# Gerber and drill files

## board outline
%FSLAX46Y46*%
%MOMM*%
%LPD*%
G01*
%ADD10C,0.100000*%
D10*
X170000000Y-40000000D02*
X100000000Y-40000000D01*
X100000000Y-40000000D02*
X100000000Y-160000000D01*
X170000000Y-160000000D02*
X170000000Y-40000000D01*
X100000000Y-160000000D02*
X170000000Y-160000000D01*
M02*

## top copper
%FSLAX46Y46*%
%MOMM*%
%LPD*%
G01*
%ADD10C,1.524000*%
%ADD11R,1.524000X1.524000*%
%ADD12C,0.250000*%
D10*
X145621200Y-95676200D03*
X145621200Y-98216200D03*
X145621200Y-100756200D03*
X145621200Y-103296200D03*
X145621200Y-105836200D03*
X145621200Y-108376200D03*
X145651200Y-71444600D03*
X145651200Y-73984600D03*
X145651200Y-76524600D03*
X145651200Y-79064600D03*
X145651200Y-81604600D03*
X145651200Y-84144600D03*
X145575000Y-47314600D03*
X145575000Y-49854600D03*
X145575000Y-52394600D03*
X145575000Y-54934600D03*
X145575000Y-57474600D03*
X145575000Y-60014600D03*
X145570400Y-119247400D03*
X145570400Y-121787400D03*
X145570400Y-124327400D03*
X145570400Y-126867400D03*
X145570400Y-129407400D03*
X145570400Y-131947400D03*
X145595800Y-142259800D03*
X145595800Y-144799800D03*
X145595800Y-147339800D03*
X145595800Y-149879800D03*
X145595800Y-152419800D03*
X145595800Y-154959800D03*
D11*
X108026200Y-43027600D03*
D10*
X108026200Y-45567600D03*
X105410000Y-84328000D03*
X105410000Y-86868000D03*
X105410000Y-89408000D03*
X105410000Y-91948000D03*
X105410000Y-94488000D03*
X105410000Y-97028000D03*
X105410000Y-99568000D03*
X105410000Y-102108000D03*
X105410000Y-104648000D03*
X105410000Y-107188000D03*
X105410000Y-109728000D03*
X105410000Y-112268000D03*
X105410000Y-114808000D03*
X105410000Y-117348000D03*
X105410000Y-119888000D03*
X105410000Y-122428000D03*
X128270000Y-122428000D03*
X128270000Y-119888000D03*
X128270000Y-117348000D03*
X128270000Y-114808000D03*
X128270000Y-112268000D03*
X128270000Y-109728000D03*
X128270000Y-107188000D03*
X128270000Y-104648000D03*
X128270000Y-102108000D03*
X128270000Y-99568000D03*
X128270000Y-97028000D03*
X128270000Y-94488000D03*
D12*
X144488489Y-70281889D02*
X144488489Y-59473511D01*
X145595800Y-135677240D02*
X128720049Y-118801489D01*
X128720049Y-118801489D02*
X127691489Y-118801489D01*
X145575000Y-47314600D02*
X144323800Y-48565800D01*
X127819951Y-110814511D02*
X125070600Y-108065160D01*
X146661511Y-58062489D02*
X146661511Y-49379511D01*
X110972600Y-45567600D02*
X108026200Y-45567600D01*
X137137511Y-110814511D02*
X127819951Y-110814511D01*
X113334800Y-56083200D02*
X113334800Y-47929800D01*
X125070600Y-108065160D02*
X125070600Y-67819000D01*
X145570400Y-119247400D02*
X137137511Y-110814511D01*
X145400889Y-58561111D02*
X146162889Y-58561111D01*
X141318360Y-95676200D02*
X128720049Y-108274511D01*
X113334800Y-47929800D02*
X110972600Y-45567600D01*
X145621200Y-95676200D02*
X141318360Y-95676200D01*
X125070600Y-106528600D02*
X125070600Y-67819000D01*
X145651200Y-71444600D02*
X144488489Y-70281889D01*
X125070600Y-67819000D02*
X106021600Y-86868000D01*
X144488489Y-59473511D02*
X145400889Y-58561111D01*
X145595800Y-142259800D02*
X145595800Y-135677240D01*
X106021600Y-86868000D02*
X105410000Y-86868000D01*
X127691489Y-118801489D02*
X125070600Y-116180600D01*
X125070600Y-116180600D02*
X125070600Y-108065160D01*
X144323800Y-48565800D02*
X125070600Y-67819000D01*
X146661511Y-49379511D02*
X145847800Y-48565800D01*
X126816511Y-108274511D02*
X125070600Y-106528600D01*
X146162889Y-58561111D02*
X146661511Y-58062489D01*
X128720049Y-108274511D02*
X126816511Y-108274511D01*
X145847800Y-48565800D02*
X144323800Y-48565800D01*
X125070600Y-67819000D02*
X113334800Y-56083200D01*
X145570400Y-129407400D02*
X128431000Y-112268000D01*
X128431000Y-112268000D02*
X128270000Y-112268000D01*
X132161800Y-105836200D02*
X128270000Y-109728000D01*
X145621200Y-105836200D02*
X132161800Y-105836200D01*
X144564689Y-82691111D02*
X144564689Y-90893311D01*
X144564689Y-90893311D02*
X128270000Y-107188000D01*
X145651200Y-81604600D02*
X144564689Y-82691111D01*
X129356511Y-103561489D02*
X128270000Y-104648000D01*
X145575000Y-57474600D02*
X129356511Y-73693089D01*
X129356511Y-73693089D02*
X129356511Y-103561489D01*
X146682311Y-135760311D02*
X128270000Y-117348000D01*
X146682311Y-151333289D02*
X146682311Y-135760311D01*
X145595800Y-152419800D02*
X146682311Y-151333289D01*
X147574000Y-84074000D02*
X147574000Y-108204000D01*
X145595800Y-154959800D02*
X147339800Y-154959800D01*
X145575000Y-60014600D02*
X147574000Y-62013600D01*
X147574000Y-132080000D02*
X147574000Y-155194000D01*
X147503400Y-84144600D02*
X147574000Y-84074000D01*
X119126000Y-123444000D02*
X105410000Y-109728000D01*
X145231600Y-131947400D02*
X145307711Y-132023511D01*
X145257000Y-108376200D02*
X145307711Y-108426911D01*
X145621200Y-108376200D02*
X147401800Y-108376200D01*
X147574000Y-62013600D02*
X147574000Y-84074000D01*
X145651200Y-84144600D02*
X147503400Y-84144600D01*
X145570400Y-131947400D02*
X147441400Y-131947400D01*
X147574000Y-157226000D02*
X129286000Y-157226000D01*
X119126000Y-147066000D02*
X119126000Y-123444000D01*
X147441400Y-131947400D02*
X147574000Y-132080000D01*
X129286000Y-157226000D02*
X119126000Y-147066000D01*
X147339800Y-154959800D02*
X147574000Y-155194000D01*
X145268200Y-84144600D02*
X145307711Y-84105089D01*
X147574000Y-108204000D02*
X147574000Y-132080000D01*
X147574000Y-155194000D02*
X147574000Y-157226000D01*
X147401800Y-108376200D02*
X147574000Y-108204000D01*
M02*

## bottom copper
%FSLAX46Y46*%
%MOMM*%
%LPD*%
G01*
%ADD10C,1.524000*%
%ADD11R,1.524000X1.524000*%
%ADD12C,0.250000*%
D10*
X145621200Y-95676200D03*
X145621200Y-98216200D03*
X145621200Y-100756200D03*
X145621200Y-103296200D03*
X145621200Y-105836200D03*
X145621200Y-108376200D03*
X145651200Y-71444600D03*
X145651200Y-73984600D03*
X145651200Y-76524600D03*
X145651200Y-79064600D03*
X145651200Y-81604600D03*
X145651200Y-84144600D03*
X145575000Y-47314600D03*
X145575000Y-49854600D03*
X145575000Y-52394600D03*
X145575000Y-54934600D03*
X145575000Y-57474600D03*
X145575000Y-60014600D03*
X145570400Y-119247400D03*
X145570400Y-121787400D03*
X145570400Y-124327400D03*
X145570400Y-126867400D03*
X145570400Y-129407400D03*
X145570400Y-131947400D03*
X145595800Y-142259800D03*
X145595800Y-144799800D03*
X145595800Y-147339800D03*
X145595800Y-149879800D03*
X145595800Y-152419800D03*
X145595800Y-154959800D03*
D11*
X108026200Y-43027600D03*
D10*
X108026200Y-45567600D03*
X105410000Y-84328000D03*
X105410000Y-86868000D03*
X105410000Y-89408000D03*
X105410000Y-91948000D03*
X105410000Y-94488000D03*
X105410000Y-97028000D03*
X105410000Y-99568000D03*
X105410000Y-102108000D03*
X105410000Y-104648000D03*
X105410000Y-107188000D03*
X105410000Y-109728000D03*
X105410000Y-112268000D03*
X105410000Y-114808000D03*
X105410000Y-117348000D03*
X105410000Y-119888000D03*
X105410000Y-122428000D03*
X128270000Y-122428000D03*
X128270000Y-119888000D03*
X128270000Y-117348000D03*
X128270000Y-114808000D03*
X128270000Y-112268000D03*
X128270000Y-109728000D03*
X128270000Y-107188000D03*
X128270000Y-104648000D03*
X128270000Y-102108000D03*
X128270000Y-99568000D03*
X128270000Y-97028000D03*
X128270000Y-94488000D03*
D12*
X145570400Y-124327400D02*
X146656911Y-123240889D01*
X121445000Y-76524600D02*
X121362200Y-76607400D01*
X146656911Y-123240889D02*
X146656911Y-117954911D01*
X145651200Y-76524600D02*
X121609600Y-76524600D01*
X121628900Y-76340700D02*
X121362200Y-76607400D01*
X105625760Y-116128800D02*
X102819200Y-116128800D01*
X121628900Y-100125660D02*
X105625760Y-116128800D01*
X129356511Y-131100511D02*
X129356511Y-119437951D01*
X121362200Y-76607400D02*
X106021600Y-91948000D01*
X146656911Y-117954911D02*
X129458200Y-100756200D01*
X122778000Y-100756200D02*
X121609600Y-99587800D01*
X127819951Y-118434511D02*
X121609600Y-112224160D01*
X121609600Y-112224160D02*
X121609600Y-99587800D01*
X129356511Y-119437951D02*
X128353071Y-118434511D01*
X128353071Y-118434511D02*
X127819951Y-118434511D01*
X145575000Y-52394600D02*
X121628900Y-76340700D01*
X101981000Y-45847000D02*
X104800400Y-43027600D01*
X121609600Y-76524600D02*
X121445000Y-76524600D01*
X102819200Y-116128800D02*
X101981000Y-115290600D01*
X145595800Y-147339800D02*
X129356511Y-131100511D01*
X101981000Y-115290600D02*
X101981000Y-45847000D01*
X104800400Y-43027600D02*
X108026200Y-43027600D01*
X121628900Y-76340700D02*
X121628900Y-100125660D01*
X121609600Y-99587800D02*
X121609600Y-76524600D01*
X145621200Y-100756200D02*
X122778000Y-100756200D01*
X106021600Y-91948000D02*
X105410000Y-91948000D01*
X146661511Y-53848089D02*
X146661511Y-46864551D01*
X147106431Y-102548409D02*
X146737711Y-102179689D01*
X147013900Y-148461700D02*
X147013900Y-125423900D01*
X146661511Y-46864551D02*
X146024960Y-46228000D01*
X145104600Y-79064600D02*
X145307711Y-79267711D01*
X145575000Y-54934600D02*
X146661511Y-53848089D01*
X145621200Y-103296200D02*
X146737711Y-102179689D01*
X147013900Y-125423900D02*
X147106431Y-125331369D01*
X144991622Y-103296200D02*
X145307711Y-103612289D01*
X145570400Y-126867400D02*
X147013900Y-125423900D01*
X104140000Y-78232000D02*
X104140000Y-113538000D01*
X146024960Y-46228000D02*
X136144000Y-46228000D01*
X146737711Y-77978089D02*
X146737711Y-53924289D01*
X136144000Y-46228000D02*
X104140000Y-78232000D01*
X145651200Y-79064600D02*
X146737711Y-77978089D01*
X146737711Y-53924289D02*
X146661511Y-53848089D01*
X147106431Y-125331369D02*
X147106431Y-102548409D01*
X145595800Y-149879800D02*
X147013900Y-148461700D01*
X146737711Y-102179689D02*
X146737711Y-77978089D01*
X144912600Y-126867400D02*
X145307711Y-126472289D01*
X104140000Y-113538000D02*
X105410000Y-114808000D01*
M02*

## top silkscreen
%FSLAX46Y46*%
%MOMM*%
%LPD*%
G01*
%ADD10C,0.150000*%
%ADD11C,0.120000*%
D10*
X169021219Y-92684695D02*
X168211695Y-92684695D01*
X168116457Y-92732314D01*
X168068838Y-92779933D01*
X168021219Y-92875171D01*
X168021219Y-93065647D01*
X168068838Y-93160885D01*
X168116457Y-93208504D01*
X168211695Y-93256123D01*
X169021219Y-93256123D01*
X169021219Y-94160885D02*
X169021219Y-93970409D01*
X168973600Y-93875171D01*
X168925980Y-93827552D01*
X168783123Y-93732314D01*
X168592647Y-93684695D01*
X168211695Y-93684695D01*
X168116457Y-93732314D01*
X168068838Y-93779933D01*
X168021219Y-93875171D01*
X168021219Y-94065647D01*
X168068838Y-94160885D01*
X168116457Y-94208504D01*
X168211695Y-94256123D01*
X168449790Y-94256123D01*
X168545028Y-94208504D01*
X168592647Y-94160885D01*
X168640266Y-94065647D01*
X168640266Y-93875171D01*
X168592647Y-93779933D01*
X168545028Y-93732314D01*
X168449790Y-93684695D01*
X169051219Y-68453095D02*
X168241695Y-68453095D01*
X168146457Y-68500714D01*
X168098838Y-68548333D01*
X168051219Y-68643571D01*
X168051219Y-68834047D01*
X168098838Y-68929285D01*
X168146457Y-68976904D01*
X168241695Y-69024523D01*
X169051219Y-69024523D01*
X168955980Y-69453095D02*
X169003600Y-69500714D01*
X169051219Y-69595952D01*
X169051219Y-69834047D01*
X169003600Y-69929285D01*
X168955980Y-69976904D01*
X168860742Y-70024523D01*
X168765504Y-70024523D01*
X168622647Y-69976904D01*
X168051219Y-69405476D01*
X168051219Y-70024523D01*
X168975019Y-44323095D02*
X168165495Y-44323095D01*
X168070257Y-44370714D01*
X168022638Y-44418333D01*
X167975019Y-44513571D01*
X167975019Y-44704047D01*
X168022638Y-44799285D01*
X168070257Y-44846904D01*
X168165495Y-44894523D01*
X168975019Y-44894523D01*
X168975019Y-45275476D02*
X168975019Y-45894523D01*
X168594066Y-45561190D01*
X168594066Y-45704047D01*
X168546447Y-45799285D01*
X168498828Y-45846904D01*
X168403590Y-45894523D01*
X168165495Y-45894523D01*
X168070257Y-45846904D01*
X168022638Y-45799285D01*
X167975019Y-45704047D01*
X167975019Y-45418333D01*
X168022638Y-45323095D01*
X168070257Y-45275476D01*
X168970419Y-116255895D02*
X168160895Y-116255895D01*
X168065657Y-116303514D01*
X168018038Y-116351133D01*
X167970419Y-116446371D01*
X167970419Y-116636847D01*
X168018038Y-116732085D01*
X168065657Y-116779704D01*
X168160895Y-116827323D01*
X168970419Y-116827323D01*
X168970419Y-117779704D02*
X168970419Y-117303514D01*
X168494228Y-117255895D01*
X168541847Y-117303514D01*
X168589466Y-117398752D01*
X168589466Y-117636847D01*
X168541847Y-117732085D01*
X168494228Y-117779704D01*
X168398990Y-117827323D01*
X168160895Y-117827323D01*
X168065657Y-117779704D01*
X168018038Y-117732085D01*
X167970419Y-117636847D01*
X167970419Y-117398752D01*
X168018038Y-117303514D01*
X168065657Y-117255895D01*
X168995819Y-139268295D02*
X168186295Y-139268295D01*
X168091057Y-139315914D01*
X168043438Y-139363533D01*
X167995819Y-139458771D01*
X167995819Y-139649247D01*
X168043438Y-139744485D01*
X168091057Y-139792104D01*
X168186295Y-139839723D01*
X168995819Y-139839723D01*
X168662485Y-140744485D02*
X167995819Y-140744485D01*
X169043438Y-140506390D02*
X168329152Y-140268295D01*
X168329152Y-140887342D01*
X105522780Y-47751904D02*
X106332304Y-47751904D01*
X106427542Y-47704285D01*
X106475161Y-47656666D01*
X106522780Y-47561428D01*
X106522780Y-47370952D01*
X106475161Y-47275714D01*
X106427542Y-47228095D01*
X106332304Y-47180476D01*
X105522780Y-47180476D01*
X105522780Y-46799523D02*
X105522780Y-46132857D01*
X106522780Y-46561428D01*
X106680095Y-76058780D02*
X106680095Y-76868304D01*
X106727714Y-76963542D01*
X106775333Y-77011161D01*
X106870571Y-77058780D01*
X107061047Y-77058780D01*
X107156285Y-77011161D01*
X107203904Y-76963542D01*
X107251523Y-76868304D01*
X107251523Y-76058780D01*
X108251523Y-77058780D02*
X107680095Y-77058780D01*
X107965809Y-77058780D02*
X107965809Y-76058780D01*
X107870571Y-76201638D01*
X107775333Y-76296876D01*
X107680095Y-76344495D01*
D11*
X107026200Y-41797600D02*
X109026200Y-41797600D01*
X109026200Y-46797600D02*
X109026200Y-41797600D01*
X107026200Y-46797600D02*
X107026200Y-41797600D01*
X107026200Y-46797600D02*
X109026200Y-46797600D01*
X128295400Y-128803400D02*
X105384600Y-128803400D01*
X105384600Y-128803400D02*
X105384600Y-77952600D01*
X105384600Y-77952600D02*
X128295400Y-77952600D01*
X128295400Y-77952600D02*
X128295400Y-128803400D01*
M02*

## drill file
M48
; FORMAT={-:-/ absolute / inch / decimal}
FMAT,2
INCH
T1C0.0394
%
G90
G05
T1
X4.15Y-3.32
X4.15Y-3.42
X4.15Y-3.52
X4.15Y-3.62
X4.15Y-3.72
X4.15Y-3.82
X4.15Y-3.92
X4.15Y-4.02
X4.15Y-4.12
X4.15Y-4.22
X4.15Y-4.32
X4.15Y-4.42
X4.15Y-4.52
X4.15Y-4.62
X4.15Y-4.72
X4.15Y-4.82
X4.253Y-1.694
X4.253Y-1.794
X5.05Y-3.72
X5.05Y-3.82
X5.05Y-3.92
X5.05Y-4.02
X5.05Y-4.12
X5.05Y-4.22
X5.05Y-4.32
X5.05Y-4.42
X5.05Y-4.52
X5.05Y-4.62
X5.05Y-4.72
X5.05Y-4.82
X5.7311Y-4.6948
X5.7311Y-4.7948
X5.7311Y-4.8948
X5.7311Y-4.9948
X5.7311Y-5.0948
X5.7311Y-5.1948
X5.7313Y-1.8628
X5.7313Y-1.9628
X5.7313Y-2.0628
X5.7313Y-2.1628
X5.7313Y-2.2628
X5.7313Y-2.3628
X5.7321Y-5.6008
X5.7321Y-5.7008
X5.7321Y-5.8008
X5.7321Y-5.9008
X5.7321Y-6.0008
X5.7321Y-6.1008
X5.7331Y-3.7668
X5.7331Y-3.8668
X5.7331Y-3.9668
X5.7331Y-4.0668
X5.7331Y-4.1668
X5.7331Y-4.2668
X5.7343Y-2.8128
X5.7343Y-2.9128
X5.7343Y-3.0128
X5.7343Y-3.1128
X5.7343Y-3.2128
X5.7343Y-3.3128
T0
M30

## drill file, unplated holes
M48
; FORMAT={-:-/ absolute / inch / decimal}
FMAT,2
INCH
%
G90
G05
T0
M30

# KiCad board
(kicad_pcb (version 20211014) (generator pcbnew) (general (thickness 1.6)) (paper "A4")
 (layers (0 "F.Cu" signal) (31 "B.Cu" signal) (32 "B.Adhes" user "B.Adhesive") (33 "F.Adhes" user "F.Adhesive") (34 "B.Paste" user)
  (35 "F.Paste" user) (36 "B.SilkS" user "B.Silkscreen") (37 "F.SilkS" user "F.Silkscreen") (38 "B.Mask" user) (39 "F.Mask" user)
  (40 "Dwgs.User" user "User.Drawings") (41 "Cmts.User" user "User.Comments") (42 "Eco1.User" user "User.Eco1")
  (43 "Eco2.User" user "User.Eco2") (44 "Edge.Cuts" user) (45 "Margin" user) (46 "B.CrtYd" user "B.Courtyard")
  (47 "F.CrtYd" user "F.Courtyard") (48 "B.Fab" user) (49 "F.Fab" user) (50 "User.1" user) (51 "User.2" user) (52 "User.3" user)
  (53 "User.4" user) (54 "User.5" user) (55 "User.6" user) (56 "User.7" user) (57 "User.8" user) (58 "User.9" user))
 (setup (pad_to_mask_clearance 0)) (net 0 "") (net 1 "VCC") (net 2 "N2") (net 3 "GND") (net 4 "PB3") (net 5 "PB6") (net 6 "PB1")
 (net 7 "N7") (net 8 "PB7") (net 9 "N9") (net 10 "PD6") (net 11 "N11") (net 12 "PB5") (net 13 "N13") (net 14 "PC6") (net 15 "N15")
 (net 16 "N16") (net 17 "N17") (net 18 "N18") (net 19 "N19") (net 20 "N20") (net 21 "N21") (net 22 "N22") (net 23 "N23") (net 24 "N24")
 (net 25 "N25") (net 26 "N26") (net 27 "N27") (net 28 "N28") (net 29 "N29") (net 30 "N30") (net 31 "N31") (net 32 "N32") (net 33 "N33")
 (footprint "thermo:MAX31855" (layer "F.Cu") (at 155.6212 101.6762 -90)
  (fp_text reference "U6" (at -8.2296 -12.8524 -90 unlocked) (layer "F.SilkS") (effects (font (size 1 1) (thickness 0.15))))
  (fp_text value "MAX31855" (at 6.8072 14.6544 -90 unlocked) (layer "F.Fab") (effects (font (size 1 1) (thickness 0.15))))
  (pad "1" thru_hole circle (at -6 10 270) (size 1.524 1.524) (drill 1) (layers *.Cu *.Mask) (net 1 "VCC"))
  (pad "2" thru_hole circle (at -3.46 10 270) (size 1.524 1.524) (drill 1) (layers *.Cu *.Mask) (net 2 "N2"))
  (pad "3" thru_hole circle (at -0.92 10 270) (size 1.524 1.524) (drill 1) (layers *.Cu *.Mask) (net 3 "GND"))
  (pad "4" thru_hole circle (at 1.62 10 270) (size 1.524 1.524) (drill 1) (layers *.Cu *.Mask) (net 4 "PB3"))
  (pad "5" thru_hole circle (at 4.16 10 270) (size 1.524 1.524) (drill 1) (layers *.Cu *.Mask) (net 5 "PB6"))
  (pad "6" thru_hole circle (at 6.7 10 270) (size 1.524 1.524) (drill 1) (layers *.Cu *.Mask) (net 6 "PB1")))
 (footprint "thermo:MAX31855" (layer "F.Cu") (at 155.6512 77.4446 -90)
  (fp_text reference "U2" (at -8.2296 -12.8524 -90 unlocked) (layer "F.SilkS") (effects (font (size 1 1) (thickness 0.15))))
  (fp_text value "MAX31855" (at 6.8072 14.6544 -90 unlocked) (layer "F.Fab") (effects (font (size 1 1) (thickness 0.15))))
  (pad "1" thru_hole circle (at -6 10 270) (size 1.524 1.524) (drill 1) (layers *.Cu *.Mask) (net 1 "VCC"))
  (pad "2" thru_hole circle (at -3.46 10 270) (size 1.524 1.524) (drill 1) (layers *.Cu *.Mask) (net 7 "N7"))
  (pad "3" thru_hole circle (at -0.92 10 270) (size 1.524 1.524) (drill 1) (layers *.Cu *.Mask) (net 3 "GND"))
  (pad "4" thru_hole circle (at 1.62 10 270) (size 1.524 1.524) (drill 1) (layers *.Cu *.Mask) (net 4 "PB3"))
  (pad "5" thru_hole circle (at 4.16 10 270) (size 1.524 1.524) (drill 1) (layers *.Cu *.Mask) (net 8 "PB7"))
  (pad "6" thru_hole circle (at 6.7 10 270) (size 1.524 1.524) (drill 1) (layers *.Cu *.Mask) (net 6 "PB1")))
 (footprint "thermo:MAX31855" (layer "F.Cu") (at 155.575 53.3146 -90)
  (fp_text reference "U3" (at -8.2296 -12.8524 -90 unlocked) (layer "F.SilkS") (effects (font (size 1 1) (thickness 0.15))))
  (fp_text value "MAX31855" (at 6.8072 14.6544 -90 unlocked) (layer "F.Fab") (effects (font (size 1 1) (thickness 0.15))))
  (pad "1" thru_hole circle (at -6 10 270) (size 1.524 1.524) (drill 1) (layers *.Cu *.Mask) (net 1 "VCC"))
  (pad "2" thru_hole circle (at -3.46 10 270) (size 1.524 1.524) (drill 1) (layers *.Cu *.Mask) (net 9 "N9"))
  (pad "3" thru_hole circle (at -0.92 10 270) (size 1.524 1.524) (drill 1) (layers *.Cu *.Mask) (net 3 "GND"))
  (pad "4" thru_hole circle (at 1.62 10 270) (size 1.524 1.524) (drill 1) (layers *.Cu *.Mask) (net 4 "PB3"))
  (pad "5" thru_hole circle (at 4.16 10 270) (size 1.524 1.524) (drill 1) (layers *.Cu *.Mask) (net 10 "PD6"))
  (pad "6" thru_hole circle (at 6.7 10 270) (size 1.524 1.524) (drill 1) (layers *.Cu *.Mask) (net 6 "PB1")))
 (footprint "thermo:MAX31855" (layer "F.Cu") (at 155.5704 125.2474 -90)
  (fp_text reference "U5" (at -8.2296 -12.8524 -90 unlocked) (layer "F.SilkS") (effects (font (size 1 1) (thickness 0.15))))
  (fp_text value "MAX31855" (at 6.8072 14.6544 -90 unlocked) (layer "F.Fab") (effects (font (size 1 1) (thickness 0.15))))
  (pad "1" thru_hole circle (at -6 10 270) (size 1.524 1.524) (drill 1) (layers *.Cu *.Mask) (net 1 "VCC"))
  (pad "2" thru_hole circle (at -3.46 10 270) (size 1.524 1.524) (drill 1) (layers *.Cu *.Mask) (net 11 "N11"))
  (pad "3" thru_hole circle (at -0.92 10 270) (size 1.524 1.524) (drill 1) (layers *.Cu *.Mask) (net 3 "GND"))
  (pad "4" thru_hole circle (at 1.62 10 270) (size 1.524 1.524) (drill 1) (layers *.Cu *.Mask) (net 4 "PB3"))
  (pad "5" thru_hole circle (at 4.16 10 270) (size 1.524 1.524) (drill 1) (layers *.Cu *.Mask) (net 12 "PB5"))
  (pad "6" thru_hole circle (at 6.7 10 270) (size 1.524 1.524) (drill 1) (layers *.Cu *.Mask) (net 6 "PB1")))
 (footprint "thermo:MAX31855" (layer "F.Cu") (at 155.5958 148.2598 -90)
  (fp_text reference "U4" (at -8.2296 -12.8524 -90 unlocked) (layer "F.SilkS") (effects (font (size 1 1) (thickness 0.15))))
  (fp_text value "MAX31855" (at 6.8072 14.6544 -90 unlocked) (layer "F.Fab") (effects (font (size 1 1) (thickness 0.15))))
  (pad "1" thru_hole circle (at -6 10 270) (size 1.524 1.524) (drill 1) (layers *.Cu *.Mask) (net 1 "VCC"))
  (pad "2" thru_hole circle (at -3.46 10 270) (size 1.524 1.524) (drill 1) (layers *.Cu *.Mask) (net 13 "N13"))
  (pad "3" thru_hole circle (at -0.92 10 270) (size 1.524 1.524) (drill 1) (layers *.Cu *.Mask) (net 3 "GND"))
  (pad "4" thru_hole circle (at 1.62 10 270) (size 1.524 1.524) (drill 1) (layers *.Cu *.Mask) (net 4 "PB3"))
  (pad "5" thru_hole circle (at 4.16 10 270) (size 1.524 1.524) (drill 1) (layers *.Cu *.Mask) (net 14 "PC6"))
  (pad "6" thru_hole circle (at 6.7 10 270) (size 1.524 1.524) (drill 1) (layers *.Cu *.Mask) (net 6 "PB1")))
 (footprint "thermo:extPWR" (layer "F.Cu") (at 108.0262 44.2976 90)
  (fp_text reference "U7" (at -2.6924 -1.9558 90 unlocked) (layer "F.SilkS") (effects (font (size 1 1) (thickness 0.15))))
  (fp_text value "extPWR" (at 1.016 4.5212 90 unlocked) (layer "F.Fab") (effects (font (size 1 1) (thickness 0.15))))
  (fp_line (start 2.5 -1) (end 2.5 1) (layer "F.SilkS") (width 0.12))
  (fp_line (start -2.5 1) (end 2.5 1) (layer "F.SilkS") (width 0.12))
  (fp_line (start -2.5 -1) (end 2.5 -1) (layer "F.SilkS") (width 0.12))
  (fp_line (start -2.5 -1) (end -2.5 1) (layer "F.SilkS") (width 0.12))
  (pad "1" thru_hole rect (at 1.27 0 90) (size 1.524 1.524) (drill 1) (layers *.Cu *.Mask) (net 3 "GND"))
  (pad "2" thru_hole circle (at -1.27 0 90) (size 1.524 1.524) (drill 1) (layers *.Cu *.Mask) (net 1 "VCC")))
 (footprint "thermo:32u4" (layer "F.Cu") (at 116.84 103.378)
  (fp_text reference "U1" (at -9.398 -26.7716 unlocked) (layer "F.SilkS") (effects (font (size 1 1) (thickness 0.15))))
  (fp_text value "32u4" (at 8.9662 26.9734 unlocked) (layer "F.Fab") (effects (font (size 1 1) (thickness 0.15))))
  (fp_poly
   (pts (xy 11.4554 25.4254) (xy -11.4554 25.4254) (xy -11.4554 -25.4254) (xy 11.4554 -25.4254)) (layer "F.SilkS") (width 0.12) (fill none))
  (pad "1" thru_hole circle (at -11.43 -19.05) (size 1.524 1.524) (drill 1) (layers *.Cu *.Mask) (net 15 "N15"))
  (pad "2" thru_hole circle (at -11.43 -16.51) (size 1.524 1.524) (drill 1) (layers *.Cu *.Mask) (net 1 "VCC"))
  (pad "3" thru_hole circle (at -11.43 -13.97) (size 1.524 1.524) (drill 1) (layers *.Cu *.Mask) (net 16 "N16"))
  (pad "4" thru_hole circle (at -11.43 -11.43) (size 1.524 1.524) (drill 1) (layers *.Cu *.Mask) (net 3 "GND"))
  (pad "5" thru_hole circle (at -11.43 -8.89) (size 1.524 1.524) (drill 1) (layers *.Cu *.Mask) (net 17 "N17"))
  (pad "6" thru_hole circle (at -11.43 -6.35) (size 1.524 1.524) (drill 1) (layers *.Cu *.Mask) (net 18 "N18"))
  (pad "7" thru_hole circle (at -11.43 -3.81) (size 1.524 1.524) (drill 1) (layers *.Cu *.Mask) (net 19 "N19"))
  (pad "8" thru_hole circle (at -11.43 -1.27) (size 1.524 1.524) (drill 1) (layers *.Cu *.Mask) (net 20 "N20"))
  (pad "9" thru_hole circle (at -11.43 1.27) (size 1.524 1.524) (drill 1) (layers *.Cu *.Mask) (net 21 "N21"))
  (pad "10" thru_hole circle (at -11.43 3.81) (size 1.524 1.524) (drill 1) (layers *.Cu *.Mask) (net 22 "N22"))
  (pad "11" thru_hole circle (at -11.43 6.35) (size 1.524 1.524) (drill 1) (layers *.Cu *.Mask) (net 6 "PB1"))
  (pad "12" thru_hole circle (at -11.43 8.89) (size 1.524 1.524) (drill 1) (layers *.Cu *.Mask) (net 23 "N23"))
  (pad "13" thru_hole circle (at -11.43 11.43) (size 1.524 1.524) (drill 1) (layers *.Cu *.Mask) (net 4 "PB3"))
  (pad "14" thru_hole circle (at -11.43 13.97) (size 1.524 1.524) (drill 1) (layers *.Cu *.Mask) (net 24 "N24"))
  (pad "15" thru_hole circle (at -11.43 16.51) (size 1.524 1.524) (drill 1) (layers *.Cu *.Mask) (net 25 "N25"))
  (pad "16" thru_hole circle (at -11.43 19.05) (size 1.524 1.524) (drill 1) (layers *.Cu *.Mask) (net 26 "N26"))
  (pad "19" thru_hole circle (at 11.43 19.05) (size 1.524 1.524) (drill 1) (layers *.Cu *.Mask) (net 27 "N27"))
  (pad "20" thru_hole circle (at 11.43 16.51) (size 1.524 1.524) (drill 1) (layers *.Cu *.Mask) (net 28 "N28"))
  (pad "21" thru_hole circle (at 11.43 13.97) (size 1.524 1.524) (drill 1) (layers *.Cu *.Mask) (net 14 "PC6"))
  (pad "22" thru_hole circle (at 11.43 11.43) (size 1.524 1.524) (drill 1) (layers *.Cu *.Mask) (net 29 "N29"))
  (pad "23" thru_hole circle (at 11.43 8.89) (size 1.524 1.524) (drill 1) (layers *.Cu *.Mask) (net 12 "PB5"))
  (pad "24" thru_hole circle (at 11.43 6.35) (size 1.524 1.524) (drill 1) (layers *.Cu *.Mask) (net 5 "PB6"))
  (pad "25" thru_hole circle (at 11.43 3.81) (size 1.524 1.524) (drill 1) (layers *.Cu *.Mask) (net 8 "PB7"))
  (pad "26" thru_hole circle (at 11.43 1.27) (size 1.524 1.524) (drill 1) (layers *.Cu *.Mask) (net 10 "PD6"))
  (pad "27" thru_hole circle (at 11.43 -1.27) (size 1.524 1.524) (drill 1) (layers *.Cu *.Mask) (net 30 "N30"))
  (pad "28" thru_hole circle (at 11.43 -3.81) (size 1.524 1.524) (drill 1) (layers *.Cu *.Mask) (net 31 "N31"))
  (pad "29" thru_hole circle (at 11.43 -6.35) (size 1.524 1.524) (drill 1) (layers *.Cu *.Mask) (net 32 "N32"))
  (pad "30" thru_hole circle (at 11.43 -8.89) (size 1.524 1.524) (drill 1) (layers *.Cu *.Mask) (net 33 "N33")))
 (gr_line (start 170 40) (end 100 40) (layer "Edge.Cuts") (width 0.1))
 (gr_line (start 100 40) (end 100 160) (layer "Edge.Cuts") (width 0.1))
 (gr_line (start 170 160) (end 170 40) (layer "Edge.Cuts") (width 0.1))
 (gr_line (start 100 160) (end 170 160) (layer "Edge.Cuts") (width 0.1))
 (segment (start 144.488489 70.281889) (end 144.488489 59.473511) (width 0.25) (layer "F.Cu") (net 1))
 (segment (start 145.5958 135.67724) (end 128.720049 118.801489) (width 0.25) (layer "F.Cu") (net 1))
 (segment (start 128.720049 118.801489) (end 127.691489 118.801489) (width 0.25) (layer "F.Cu") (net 1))
 (segment (start 145.575 47.3146) (end 144.3238 48.5658) (width 0.25) (layer "F.Cu") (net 1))
 (segment (start 127.819951 110.814511) (end 125.0706 108.06516) (width 0.25) (layer "F.Cu") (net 1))
 (segment (start 146.661511 58.062489) (end 146.661511 49.379511) (width 0.25) (layer "F.Cu") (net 1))
 (segment (start 110.9726 45.5676) (end 108.0262 45.5676) (width 0.25) (layer "F.Cu") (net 1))
 (segment (start 137.137511 110.814511) (end 127.819951 110.814511) (width 0.25) (layer "F.Cu") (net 1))
 (segment (start 113.3348 56.0832) (end 113.3348 47.9298) (width 0.25) (layer "F.Cu") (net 1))
 (segment (start 125.0706 108.06516) (end 125.0706 67.819) (width 0.25) (layer "F.Cu") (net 1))
 (segment (start 145.5704 119.2474) (end 137.137511 110.814511) (width 0.25) (layer "F.Cu") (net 1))
 (segment (start 145.400889 58.561111) (end 146.162889 58.561111) (width 0.25) (layer "F.Cu") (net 1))
 (segment (start 141.31836 95.6762) (end 128.720049 108.274511) (width 0.25) (layer "F.Cu") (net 1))
 (segment (start 113.3348 47.9298) (end 110.9726 45.5676) (width 0.25) (layer "F.Cu") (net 1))
 (segment (start 145.6212 95.6762) (end 141.31836 95.6762) (width 0.25) (layer "F.Cu") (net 1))
 (segment (start 125.0706 106.5286) (end 125.0706 67.819) (width 0.25) (layer "F.Cu") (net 1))
 (segment (start 145.6512 71.4446) (end 144.488489 70.281889) (width 0.25) (layer "F.Cu") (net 1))
 (segment (start 125.0706 67.819) (end 106.0216 86.868) (width 0.25) (layer "F.Cu") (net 1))
 (segment (start 144.488489 59.473511) (end 145.400889 58.561111) (width 0.25) (layer "F.Cu") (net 1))
 (segment (start 145.5958 142.2598) (end 145.5958 135.67724) (width 0.25) (layer "F.Cu") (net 1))
 (segment (start 106.0216 86.868) (end 105.41 86.868) (width 0.25) (layer "F.Cu") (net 1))
 (segment (start 127.691489 118.801489) (end 125.0706 116.1806) (width 0.25) (layer "F.Cu") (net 1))
 (segment (start 125.0706 116.1806) (end 125.0706 108.06516) (width 0.25) (layer "F.Cu") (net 1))
 (segment (start 144.3238 48.5658) (end 125.0706 67.819) (width 0.25) (layer "F.Cu") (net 1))
 (segment (start 146.661511 49.379511) (end 145.8478 48.5658) (width 0.25) (layer "F.Cu") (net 1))
 (segment (start 126.816511 108.274511) (end 125.0706 106.5286) (width 0.25) (layer "F.Cu") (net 1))
 (segment (start 146.162889 58.561111) (end 146.661511 58.062489) (width 0.25) (layer "F.Cu") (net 1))
 (segment (start 128.720049 108.274511) (end 126.816511 108.274511) (width 0.25) (layer "F.Cu") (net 1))
 (segment (start 145.8478 48.5658) (end 144.3238 48.5658) (width 0.25) (layer "F.Cu") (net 1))
 (segment (start 125.0706 67.819) (end 113.3348 56.0832) (width 0.25) (layer "F.Cu") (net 1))
 (segment (start 145.5704 124.3274) (end 146.656911 123.240889) (width 0.25) (layer "B.Cu") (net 3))
 (segment (start 121.445 76.5246) (end 121.3622 76.6074) (width 0.25) (layer "B.Cu") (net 3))
 (segment (start 146.656911 123.240889) (end 146.656911 117.954911) (width 0.25) (layer "B.Cu") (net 3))
 (segment (start 145.6512 76.5246) (end 121.6096 76.5246) (width 0.25) (layer "B.Cu") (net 3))
 (segment (start 121.6289 76.3407) (end 121.3622 76.6074) (width 0.25) (layer "B.Cu") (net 3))
 (segment (start 105.62576 116.1288) (end 102.8192 116.1288) (width 0.25) (layer "B.Cu") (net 3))
 (segment (start 121.6289 100.12566) (end 105.62576 116.1288) (width 0.25) (layer "B.Cu") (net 3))
 (segment (start 129.356511 131.100511) (end 129.356511 119.437951) (width 0.25) (layer "B.Cu") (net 3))
 (segment (start 121.3622 76.6074) (end 106.0216 91.948) (width 0.25) (layer "B.Cu") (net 3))
 (segment (start 146.656911 117.954911) (end 129.4582 100.7562) (width 0.25) (layer "B.Cu") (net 3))
 (segment (start 122.778 100.7562) (end 121.6096 99.5878) (width 0.25) (layer "B.Cu") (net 3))
 (segment (start 127.819951 118.434511) (end 121.6096 112.22416) (width 0.25) (layer "B.Cu") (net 3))
 (segment (start 121.6096 112.22416) (end 121.6096 99.5878) (width 0.25) (layer "B.Cu") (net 3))
 (segment (start 129.356511 119.437951) (end 128.353071 118.434511) (width 0.25) (layer "B.Cu") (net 3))
 (segment (start 128.353071 118.434511) (end 127.819951 118.434511) (width 0.25) (layer "B.Cu") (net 3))
 (segment (start 145.575 52.3946) (end 121.6289 76.3407) (width 0.25) (layer "B.Cu") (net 3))
 (segment (start 101.981 45.847) (end 104.8004 43.0276) (width 0.25) (layer "B.Cu") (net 3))
 (segment (start 121.6096 76.5246) (end 121.445 76.5246) (width 0.25) (layer "B.Cu") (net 3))
 (segment (start 102.8192 116.1288) (end 101.981 115.2906) (width 0.25) (layer "B.Cu") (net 3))
 (segment (start 145.5958 147.3398) (end 129.356511 131.100511) (width 0.25) (layer "B.Cu") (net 3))
 (segment (start 101.981 115.2906) (end 101.981 45.847) (width 0.25) (layer "B.Cu") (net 3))
 (segment (start 104.8004 43.0276) (end 108.0262 43.0276) (width 0.25) (layer "B.Cu") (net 3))
 (segment (start 121.6289 76.3407) (end 121.6289 100.12566) (width 0.25) (layer "B.Cu") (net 3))
 (segment (start 121.6096 99.5878) (end 121.6096 76.5246) (width 0.25) (layer "B.Cu") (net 3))
 (segment (start 145.6212 100.7562) (end 122.778 100.7562) (width 0.25) (layer "B.Cu") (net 3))
 (segment (start 106.0216 91.948) (end 105.41 91.948) (width 0.25) (layer "B.Cu") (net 3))
 (segment (start 145.5704 129.4074) (end 128.431 112.268) (width 0.25) (layer "F.Cu") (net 12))
 (segment (start 128.431 112.268) (end 128.27 112.268) (width 0.25) (layer "F.Cu") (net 12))
 (segment (start 132.1618 105.8362) (end 128.27 109.728) (width 0.25) (layer "F.Cu") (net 5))
 (segment (start 145.6212 105.8362) (end 132.1618 105.8362) (width 0.25) (layer "F.Cu") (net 5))
 (segment (start 144.564689 82.691111) (end 144.564689 90.893311) (width 0.25) (layer "F.Cu") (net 8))
 (segment (start 144.564689 90.893311) (end 128.27 107.188) (width 0.25) (layer "F.Cu") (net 8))
 (segment (start 145.6512 81.6046) (end 144.564689 82.691111) (width 0.25) (layer "F.Cu") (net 8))
 (segment (start 129.356511 103.561489) (end 128.27 104.648) (width 0.25) (layer "F.Cu") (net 10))
 (segment (start 145.575 57.4746) (end 129.356511 73.693089) (width 0.25) (layer "F.Cu") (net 10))
 (segment (start 129.356511 73.693089) (end 129.356511 103.561489) (width 0.25) (layer "F.Cu") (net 10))
 (segment (start 146.661511 53.848089) (end 146.661511 46.864551) (width 0.25) (layer "B.Cu") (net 4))
 (segment (start 147.106431 102.548409) (end 146.737711 102.179689) (width 0.25) (layer "B.Cu") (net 4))
 (segment (start 147.0139 148.4617) (end 147.0139 125.4239) (width 0.25) (layer "B.Cu") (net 4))
 (segment (start 146.661511 46.864551) (end 146.02496 46.228) (width 0.25) (layer "B.Cu") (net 4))
 (segment (start 145.1046 79.0646) (end 145.307711 79.267711) (width 0.25) (layer "B.Cu") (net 4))
 (segment (start 145.575 54.9346) (end 146.661511 53.848089) (width 0.25) (layer "B.Cu") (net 4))
 (segment (start 145.6212 103.2962) (end 146.737711 102.179689) (width 0.25) (layer "B.Cu") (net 4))
 (segment (start 147.0139 125.4239) (end 147.106431 125.331369) (width 0.25) (layer "B.Cu") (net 4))
 (segment (start 144.991622 103.2962) (end 145.307711 103.612289) (width 0.25) (layer "B.Cu") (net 4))
 (segment (start 145.5704 126.8674) (end 147.0139 125.4239) (width 0.25) (layer "B.Cu") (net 4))
 (segment (start 104.14 78.232) (end 104.14 113.538) (width 0.25) (layer "B.Cu") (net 4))
 (segment (start 146.02496 46.228) (end 136.144 46.228) (width 0.25) (layer "B.Cu") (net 4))
 (segment (start 146.737711 77.978089) (end 146.737711 53.924289) (width 0.25) (layer "B.Cu") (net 4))
 (segment (start 136.144 46.228) (end 104.14 78.232) (width 0.25) (layer "B.Cu") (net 4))
 (segment (start 145.6512 79.0646) (end 146.737711 77.978089) (width 0.25) (layer "B.Cu") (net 4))
 (segment (start 146.737711 53.924289) (end 146.661511 53.848089) (width 0.25) (layer "B.Cu") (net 4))
 (segment (start 147.106431 125.331369) (end 147.106431 102.548409) (width 0.25) (layer "B.Cu") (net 4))
 (segment (start 145.5958 149.8798) (end 147.0139 148.4617) (width 0.25) (layer "B.Cu") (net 4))
 (segment (start 146.737711 102.179689) (end 146.737711 77.978089) (width 0.25) (layer "B.Cu") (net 4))
 (segment (start 144.9126 126.8674) (end 145.307711 126.472289) (width 0.25) (layer "B.Cu") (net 4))
 (segment (start 104.14 113.538) (end 105.41 114.808) (width 0.25) (layer "B.Cu") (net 4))
 (segment (start 146.682311 135.760311) (end 128.27 117.348) (width 0.25) (layer "F.Cu") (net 14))
 (segment (start 146.682311 151.333289) (end 146.682311 135.760311) (width 0.25) (layer "F.Cu") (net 14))
 (segment (start 145.5958 152.4198) (end 146.682311 151.333289) (width 0.25) (layer "F.Cu") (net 14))
 (segment (start 147.574 84.074) (end 147.574 108.204) (width 0.25) (layer "F.Cu") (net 6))
 (segment (start 145.5958 154.9598) (end 147.3398 154.9598) (width 0.25) (layer "F.Cu") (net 6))
 (segment (start 145.575 60.0146) (end 147.574 62.0136) (width 0.25) (layer "F.Cu") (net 6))
 (segment (start 147.574 132.08) (end 147.574 155.194) (width 0.25) (layer "F.Cu") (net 6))
 (segment (start 147.5034 84.1446) (end 147.574 84.074) (width 0.25) (layer "F.Cu") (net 6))
 (segment (start 119.126 123.444) (end 105.41 109.728) (width 0.25) (layer "F.Cu") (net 6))
 (segment (start 145.2316 131.9474) (end 145.307711 132.023511) (width 0.25) (layer "F.Cu") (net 6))
 (segment (start 145.257 108.3762) (end 145.307711 108.426911) (width 0.25) (layer "F.Cu") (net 6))
 (segment (start 145.6212 108.3762) (end 147.4018 108.3762) (width 0.25) (layer "F.Cu") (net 6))
 (segment (start 147.574 62.0136) (end 147.574 84.074) (width 0.25) (layer "F.Cu") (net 6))
 (segment (start 145.6512 84.1446) (end 147.5034 84.1446) (width 0.25) (layer "F.Cu") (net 6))
 (segment (start 145.5704 131.9474) (end 147.4414 131.9474) (width 0.25) (layer "F.Cu") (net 6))
 (segment (start 147.574 157.226) (end 129.286 157.226) (width 0.25) (layer "F.Cu") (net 6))
 (segment (start 119.126 147.066) (end 119.126 123.444) (width 0.25) (layer "F.Cu") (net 6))
 (segment (start 147.4414 131.9474) (end 147.574 132.08) (width 0.25) (layer "F.Cu") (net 6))
 (segment (start 129.286 157.226) (end 119.126 147.066) (width 0.25) (layer "F.Cu") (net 6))
 (segment (start 147.3398 154.9598) (end 147.574 155.194) (width 0.25) (layer "F.Cu") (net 6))
 (segment (start 145.2682 84.1446) (end 145.307711 84.105089) (width 0.25) (layer "F.Cu") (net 6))
 (segment (start 147.574 108.204) (end 147.574 132.08) (width 0.25) (layer "F.Cu") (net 6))
 (segment (start 147.574 155.194) (end 147.574 157.226) (width 0.25) (layer "F.Cu") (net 6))
 (segment (start 147.4018 108.3762) (end 147.574 108.204) (width 0.25) (layer "F.Cu") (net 6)))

